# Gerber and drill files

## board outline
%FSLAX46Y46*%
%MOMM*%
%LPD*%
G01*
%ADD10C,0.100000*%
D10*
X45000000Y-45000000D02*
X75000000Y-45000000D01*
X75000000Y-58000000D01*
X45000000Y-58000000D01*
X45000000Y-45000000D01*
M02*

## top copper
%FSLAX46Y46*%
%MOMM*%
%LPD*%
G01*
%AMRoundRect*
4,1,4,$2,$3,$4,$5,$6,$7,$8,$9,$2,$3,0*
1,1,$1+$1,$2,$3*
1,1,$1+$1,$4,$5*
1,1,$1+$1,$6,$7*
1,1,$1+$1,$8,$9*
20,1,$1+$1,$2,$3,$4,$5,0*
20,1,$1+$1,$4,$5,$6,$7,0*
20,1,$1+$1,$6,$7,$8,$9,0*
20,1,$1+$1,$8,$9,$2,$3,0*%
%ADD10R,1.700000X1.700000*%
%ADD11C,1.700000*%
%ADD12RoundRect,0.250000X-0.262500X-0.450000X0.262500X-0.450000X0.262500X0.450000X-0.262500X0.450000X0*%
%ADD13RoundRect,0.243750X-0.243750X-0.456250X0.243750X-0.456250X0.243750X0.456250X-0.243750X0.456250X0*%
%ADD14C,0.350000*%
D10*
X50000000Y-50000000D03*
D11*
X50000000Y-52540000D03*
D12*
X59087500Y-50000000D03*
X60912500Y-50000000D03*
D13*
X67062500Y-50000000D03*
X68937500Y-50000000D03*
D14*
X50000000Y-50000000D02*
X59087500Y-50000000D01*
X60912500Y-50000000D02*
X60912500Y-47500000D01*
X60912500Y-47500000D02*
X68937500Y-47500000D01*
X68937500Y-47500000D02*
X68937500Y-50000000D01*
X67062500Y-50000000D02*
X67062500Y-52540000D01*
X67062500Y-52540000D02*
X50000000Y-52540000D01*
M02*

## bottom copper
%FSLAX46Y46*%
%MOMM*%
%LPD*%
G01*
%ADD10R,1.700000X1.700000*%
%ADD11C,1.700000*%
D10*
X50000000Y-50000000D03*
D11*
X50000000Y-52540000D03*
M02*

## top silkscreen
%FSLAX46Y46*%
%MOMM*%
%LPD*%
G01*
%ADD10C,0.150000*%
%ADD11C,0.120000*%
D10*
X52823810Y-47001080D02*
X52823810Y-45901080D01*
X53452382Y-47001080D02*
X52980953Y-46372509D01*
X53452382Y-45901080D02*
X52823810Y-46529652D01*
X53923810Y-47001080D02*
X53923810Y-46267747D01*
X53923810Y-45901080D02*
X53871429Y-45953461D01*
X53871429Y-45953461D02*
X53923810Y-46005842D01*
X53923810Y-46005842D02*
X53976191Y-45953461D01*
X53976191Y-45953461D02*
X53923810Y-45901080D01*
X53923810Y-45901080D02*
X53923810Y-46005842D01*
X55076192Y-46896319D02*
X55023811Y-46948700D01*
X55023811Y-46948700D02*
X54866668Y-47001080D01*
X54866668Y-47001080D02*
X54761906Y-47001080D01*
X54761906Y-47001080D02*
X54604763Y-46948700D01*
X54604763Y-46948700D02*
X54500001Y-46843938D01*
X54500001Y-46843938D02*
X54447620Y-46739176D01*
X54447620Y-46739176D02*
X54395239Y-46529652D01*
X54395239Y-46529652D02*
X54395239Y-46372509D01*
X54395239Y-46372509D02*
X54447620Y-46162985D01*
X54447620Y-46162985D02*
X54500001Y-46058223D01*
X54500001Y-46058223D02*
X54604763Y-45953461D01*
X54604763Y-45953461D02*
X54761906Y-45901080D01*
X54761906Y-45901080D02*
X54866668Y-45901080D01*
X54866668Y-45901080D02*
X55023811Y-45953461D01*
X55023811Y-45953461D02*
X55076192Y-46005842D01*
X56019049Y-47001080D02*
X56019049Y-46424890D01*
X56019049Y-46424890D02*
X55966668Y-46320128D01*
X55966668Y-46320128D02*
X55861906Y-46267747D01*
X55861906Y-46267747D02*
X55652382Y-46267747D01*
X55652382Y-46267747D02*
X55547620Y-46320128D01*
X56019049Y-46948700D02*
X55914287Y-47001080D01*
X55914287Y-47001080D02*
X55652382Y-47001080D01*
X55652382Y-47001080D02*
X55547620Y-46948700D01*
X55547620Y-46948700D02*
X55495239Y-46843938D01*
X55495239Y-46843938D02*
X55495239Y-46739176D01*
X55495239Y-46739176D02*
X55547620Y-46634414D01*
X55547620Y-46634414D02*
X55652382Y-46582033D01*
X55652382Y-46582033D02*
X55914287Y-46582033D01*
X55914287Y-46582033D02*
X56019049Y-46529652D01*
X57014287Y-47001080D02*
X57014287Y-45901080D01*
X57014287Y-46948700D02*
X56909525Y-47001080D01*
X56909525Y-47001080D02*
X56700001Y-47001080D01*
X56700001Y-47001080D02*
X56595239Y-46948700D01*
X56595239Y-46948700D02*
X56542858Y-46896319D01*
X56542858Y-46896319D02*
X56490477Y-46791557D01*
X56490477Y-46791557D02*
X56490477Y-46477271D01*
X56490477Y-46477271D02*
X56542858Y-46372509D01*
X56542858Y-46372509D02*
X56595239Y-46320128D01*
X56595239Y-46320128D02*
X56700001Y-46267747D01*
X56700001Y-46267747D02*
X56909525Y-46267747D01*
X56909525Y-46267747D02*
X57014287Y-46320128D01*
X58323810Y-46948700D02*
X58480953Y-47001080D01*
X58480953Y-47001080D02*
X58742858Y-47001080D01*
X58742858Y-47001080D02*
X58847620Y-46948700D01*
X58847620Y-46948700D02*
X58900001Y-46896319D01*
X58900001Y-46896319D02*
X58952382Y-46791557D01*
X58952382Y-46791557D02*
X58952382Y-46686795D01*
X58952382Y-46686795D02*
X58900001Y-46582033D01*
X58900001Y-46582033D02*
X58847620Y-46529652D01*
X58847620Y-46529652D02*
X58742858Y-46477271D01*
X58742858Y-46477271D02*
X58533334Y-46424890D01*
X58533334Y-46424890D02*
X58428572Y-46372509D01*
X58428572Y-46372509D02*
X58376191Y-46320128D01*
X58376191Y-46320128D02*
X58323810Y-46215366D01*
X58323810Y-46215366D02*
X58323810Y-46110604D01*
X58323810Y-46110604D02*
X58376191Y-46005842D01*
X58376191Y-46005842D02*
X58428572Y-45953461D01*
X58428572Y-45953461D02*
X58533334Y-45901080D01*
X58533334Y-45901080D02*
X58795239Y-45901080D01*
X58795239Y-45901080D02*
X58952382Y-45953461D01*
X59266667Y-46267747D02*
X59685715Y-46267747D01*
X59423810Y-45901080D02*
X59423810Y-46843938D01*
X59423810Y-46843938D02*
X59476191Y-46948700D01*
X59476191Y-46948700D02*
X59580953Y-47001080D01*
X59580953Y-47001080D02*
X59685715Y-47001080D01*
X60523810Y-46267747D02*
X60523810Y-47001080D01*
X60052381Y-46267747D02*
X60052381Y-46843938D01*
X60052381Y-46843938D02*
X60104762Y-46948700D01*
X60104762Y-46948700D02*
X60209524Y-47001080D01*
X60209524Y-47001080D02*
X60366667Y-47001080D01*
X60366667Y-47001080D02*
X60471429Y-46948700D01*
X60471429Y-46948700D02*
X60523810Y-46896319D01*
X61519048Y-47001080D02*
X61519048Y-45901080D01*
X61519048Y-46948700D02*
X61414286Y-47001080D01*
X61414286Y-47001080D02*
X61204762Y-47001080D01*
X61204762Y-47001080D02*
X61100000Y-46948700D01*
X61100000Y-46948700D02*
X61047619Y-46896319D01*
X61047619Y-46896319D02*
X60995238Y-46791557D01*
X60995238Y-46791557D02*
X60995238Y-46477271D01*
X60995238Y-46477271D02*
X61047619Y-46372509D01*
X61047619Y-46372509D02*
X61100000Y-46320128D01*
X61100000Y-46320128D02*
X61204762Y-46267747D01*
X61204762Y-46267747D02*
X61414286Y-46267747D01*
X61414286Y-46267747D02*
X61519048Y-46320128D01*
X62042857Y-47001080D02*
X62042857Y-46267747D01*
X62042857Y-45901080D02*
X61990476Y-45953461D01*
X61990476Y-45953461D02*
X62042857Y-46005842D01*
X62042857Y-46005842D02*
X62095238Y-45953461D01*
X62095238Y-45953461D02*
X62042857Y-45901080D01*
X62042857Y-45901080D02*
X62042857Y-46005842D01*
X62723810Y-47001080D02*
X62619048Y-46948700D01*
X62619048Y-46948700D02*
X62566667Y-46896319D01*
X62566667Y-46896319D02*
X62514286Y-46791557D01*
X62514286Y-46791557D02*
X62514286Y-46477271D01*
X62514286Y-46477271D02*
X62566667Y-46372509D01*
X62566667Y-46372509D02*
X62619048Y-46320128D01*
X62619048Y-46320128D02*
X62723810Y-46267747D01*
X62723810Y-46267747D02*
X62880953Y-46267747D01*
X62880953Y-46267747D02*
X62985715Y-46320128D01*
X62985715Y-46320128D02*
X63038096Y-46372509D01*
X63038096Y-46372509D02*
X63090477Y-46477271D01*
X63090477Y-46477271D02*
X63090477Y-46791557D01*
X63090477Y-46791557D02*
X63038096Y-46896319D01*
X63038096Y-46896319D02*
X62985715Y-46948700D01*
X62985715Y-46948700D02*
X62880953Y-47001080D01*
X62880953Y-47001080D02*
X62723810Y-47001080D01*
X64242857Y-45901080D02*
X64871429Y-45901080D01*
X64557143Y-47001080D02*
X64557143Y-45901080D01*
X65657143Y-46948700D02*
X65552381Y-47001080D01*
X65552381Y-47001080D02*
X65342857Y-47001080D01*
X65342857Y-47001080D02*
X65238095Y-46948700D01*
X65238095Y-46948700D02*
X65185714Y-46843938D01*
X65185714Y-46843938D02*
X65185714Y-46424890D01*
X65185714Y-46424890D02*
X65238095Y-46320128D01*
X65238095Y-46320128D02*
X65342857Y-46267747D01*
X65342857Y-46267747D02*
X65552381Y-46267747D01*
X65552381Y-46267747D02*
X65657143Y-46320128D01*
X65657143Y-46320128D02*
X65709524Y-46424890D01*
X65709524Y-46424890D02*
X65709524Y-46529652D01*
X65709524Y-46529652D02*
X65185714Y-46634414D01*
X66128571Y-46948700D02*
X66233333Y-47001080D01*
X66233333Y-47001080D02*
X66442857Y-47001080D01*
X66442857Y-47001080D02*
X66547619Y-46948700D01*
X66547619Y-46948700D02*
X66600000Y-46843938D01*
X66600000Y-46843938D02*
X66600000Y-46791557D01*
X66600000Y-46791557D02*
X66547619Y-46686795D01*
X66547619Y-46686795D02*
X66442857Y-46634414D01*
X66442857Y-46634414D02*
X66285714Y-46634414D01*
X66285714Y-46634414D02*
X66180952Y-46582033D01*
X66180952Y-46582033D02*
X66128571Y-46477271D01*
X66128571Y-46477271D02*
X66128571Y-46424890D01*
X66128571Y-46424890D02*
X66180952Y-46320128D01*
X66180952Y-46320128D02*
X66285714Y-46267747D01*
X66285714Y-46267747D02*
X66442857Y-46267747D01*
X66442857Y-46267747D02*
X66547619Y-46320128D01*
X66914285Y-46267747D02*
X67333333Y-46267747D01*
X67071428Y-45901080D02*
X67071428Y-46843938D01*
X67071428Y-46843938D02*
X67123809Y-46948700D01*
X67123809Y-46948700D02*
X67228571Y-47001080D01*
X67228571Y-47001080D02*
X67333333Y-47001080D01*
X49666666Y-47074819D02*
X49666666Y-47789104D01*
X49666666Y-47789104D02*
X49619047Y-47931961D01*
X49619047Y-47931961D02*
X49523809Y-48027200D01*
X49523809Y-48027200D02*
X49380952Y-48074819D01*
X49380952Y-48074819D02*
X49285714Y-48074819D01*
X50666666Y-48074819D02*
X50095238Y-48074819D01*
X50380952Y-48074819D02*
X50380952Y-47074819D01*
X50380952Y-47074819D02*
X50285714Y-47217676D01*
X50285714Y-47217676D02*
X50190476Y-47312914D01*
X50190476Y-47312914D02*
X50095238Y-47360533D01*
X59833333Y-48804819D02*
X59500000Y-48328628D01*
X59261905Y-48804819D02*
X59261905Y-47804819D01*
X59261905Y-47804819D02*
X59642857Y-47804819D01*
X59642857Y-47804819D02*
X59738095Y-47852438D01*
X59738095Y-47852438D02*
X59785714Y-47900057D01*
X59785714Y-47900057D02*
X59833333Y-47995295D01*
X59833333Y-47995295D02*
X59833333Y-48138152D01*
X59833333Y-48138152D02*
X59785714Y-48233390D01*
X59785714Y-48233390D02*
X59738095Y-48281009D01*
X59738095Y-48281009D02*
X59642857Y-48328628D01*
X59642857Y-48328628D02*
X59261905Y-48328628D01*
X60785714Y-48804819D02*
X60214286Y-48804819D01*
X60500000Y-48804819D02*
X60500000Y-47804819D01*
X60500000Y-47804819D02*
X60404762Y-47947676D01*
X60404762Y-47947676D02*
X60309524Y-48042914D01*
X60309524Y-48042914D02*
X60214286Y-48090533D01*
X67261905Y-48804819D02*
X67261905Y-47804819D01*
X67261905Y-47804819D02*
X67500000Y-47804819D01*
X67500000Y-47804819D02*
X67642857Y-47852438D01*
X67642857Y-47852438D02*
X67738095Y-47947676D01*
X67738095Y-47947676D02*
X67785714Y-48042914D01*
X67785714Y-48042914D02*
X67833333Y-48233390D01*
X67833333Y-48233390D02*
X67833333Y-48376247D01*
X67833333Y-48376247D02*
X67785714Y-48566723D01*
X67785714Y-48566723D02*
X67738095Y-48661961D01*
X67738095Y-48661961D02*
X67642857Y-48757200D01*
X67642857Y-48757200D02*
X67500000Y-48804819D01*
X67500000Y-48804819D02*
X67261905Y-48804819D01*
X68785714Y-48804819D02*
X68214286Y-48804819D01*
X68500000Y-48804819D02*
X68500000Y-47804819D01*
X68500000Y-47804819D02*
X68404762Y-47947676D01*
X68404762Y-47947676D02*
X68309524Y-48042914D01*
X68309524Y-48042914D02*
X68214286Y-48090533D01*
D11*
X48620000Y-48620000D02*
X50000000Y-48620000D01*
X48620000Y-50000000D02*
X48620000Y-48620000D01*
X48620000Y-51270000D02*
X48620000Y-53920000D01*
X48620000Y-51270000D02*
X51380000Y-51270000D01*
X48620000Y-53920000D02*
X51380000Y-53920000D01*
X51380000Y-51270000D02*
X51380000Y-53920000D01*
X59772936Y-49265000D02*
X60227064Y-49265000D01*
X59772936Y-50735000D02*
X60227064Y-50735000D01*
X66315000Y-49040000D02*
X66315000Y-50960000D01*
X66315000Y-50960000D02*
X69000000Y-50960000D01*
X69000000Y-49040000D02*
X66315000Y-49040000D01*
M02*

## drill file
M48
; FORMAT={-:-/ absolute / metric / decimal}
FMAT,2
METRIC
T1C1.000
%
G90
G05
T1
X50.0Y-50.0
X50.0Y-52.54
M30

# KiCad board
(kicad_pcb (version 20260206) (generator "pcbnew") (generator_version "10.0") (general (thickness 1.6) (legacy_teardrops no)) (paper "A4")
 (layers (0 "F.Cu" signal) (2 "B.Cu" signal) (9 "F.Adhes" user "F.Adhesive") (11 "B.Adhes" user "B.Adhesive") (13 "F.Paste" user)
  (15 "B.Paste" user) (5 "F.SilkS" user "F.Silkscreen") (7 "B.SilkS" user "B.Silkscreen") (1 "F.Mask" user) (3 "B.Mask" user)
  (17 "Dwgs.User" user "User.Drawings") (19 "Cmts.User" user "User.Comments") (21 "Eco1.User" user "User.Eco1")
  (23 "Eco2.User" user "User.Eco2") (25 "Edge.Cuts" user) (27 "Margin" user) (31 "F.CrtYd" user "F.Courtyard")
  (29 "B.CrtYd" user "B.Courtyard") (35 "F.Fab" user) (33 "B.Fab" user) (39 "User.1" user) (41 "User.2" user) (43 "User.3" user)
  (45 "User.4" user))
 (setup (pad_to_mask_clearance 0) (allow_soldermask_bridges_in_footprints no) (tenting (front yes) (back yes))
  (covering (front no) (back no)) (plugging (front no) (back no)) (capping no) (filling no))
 (gr_rect (start 45 45) (end 75 58) (stroke (width 0.1) (type solid)) (fill no) (layer "Edge.Cuts"))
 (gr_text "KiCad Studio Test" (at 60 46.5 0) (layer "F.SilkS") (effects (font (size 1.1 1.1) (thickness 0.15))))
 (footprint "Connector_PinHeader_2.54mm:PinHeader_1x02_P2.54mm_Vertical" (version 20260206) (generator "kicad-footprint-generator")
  (layer "F.Cu") (at 50 50 0)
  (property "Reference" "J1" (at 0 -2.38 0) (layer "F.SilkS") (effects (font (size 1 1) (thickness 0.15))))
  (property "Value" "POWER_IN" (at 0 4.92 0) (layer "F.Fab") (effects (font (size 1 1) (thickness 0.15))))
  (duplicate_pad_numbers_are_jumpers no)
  (fp_line (start -1.38 -1.38) (end 0 -1.38) (stroke (width 0.12) (type solid)) (layer "F.SilkS"))
  (fp_line (start -1.38 0) (end -1.38 -1.38) (stroke (width 0.12) (type solid)) (layer "F.SilkS"))
  (fp_line (start -1.38 1.27) (end -1.38 3.92) (stroke (width 0.12) (type solid)) (layer "F.SilkS"))
  (fp_line (start -1.38 1.27) (end 1.38 1.27) (stroke (width 0.12) (type solid)) (layer "F.SilkS"))
  (fp_line (start -1.38 3.92) (end 1.38 3.92) (stroke (width 0.12) (type solid)) (layer "F.SilkS"))
  (fp_line (start 1.38 1.27) (end 1.38 3.92) (stroke (width 0.12) (type solid)) (layer "F.SilkS"))
  (pad "1" thru_hole rect (at 0 0) (size 1.7 1.7) (drill 1) (layers "*.Cu" "*.Mask") (remove_unused_layers no) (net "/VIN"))
  (pad "2" thru_hole circle (at 0 2.54) (size 1.7 1.7) (drill 1) (layers "*.Cu" "*.Mask") (remove_unused_layers no) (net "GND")))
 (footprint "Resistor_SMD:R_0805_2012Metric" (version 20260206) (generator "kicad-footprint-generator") (layer "F.Cu") (at 60 50 0)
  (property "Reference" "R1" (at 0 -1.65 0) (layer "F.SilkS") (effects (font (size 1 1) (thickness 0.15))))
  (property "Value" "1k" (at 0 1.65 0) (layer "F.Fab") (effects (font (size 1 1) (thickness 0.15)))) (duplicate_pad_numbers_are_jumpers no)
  (fp_line (start -0.227064 -0.735) (end 0.227064 -0.735) (stroke (width 0.12) (type solid)) (layer "F.SilkS"))
  (fp_line (start -0.227064 0.735) (end 0.227064 0.735) (stroke (width 0.12) (type solid)) (layer "F.SilkS"))
  (pad "1" smd roundrect (at -0.9125 0) (size 1.025 1.4) (layers "F.Cu" "F.Mask" "F.Paste") (roundrect_rratio 0.243902) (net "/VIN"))
  (pad "2" smd roundrect (at 0.9125 0) (size 1.025 1.4) (layers "F.Cu" "F.Mask" "F.Paste") (roundrect_rratio 0.243902) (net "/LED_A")))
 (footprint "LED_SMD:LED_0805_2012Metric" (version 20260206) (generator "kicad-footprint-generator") (layer "F.Cu") (at 68 50 0)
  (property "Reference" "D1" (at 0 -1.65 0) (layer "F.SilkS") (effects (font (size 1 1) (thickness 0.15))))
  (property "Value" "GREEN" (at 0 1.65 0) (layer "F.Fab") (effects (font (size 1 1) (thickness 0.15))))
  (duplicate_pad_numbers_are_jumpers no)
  (fp_line (start -1.685 -0.96) (end -1.685 0.96) (stroke (width 0.12) (type solid)) (layer "F.SilkS"))
  (fp_line (start -1.685 0.96) (end 1 0.96) (stroke (width 0.12) (type solid)) (layer "F.SilkS"))
  (fp_line (start 1 -0.96) (end -1.685 -0.96) (stroke (width 0.12) (type solid)) (layer "F.SilkS"))
  (pad "1" smd roundrect (at -0.9375 0) (size 0.975 1.4) (layers "F.Cu" "F.Mask" "F.Paste") (roundrect_rratio 0.25) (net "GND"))
  (pad "2" smd roundrect (at 0.9375 0) (size 0.975 1.4) (layers "F.Cu" "F.Mask" "F.Paste") (roundrect_rratio 0.25) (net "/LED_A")))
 (segment (start 50 50) (end 59.0875 50) (width 0.35) (layer "F.Cu") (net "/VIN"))
 (segment (start 60.9125 50) (end 60.9125 47.5) (width 0.35) (layer "F.Cu") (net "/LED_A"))
 (segment (start 60.9125 47.5) (end 68.9375 47.5) (width 0.35) (layer "F.Cu") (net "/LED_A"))
 (segment (start 68.9375 47.5) (end 68.9375 50) (width 0.35) (layer "F.Cu") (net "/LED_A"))
 (segment (start 67.0625 50) (end 67.0625 52.54) (width 0.35) (layer "F.Cu") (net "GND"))
 (segment (start 67.0625 52.54) (end 50 52.54) (width 0.35) (layer "F.Cu") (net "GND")))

